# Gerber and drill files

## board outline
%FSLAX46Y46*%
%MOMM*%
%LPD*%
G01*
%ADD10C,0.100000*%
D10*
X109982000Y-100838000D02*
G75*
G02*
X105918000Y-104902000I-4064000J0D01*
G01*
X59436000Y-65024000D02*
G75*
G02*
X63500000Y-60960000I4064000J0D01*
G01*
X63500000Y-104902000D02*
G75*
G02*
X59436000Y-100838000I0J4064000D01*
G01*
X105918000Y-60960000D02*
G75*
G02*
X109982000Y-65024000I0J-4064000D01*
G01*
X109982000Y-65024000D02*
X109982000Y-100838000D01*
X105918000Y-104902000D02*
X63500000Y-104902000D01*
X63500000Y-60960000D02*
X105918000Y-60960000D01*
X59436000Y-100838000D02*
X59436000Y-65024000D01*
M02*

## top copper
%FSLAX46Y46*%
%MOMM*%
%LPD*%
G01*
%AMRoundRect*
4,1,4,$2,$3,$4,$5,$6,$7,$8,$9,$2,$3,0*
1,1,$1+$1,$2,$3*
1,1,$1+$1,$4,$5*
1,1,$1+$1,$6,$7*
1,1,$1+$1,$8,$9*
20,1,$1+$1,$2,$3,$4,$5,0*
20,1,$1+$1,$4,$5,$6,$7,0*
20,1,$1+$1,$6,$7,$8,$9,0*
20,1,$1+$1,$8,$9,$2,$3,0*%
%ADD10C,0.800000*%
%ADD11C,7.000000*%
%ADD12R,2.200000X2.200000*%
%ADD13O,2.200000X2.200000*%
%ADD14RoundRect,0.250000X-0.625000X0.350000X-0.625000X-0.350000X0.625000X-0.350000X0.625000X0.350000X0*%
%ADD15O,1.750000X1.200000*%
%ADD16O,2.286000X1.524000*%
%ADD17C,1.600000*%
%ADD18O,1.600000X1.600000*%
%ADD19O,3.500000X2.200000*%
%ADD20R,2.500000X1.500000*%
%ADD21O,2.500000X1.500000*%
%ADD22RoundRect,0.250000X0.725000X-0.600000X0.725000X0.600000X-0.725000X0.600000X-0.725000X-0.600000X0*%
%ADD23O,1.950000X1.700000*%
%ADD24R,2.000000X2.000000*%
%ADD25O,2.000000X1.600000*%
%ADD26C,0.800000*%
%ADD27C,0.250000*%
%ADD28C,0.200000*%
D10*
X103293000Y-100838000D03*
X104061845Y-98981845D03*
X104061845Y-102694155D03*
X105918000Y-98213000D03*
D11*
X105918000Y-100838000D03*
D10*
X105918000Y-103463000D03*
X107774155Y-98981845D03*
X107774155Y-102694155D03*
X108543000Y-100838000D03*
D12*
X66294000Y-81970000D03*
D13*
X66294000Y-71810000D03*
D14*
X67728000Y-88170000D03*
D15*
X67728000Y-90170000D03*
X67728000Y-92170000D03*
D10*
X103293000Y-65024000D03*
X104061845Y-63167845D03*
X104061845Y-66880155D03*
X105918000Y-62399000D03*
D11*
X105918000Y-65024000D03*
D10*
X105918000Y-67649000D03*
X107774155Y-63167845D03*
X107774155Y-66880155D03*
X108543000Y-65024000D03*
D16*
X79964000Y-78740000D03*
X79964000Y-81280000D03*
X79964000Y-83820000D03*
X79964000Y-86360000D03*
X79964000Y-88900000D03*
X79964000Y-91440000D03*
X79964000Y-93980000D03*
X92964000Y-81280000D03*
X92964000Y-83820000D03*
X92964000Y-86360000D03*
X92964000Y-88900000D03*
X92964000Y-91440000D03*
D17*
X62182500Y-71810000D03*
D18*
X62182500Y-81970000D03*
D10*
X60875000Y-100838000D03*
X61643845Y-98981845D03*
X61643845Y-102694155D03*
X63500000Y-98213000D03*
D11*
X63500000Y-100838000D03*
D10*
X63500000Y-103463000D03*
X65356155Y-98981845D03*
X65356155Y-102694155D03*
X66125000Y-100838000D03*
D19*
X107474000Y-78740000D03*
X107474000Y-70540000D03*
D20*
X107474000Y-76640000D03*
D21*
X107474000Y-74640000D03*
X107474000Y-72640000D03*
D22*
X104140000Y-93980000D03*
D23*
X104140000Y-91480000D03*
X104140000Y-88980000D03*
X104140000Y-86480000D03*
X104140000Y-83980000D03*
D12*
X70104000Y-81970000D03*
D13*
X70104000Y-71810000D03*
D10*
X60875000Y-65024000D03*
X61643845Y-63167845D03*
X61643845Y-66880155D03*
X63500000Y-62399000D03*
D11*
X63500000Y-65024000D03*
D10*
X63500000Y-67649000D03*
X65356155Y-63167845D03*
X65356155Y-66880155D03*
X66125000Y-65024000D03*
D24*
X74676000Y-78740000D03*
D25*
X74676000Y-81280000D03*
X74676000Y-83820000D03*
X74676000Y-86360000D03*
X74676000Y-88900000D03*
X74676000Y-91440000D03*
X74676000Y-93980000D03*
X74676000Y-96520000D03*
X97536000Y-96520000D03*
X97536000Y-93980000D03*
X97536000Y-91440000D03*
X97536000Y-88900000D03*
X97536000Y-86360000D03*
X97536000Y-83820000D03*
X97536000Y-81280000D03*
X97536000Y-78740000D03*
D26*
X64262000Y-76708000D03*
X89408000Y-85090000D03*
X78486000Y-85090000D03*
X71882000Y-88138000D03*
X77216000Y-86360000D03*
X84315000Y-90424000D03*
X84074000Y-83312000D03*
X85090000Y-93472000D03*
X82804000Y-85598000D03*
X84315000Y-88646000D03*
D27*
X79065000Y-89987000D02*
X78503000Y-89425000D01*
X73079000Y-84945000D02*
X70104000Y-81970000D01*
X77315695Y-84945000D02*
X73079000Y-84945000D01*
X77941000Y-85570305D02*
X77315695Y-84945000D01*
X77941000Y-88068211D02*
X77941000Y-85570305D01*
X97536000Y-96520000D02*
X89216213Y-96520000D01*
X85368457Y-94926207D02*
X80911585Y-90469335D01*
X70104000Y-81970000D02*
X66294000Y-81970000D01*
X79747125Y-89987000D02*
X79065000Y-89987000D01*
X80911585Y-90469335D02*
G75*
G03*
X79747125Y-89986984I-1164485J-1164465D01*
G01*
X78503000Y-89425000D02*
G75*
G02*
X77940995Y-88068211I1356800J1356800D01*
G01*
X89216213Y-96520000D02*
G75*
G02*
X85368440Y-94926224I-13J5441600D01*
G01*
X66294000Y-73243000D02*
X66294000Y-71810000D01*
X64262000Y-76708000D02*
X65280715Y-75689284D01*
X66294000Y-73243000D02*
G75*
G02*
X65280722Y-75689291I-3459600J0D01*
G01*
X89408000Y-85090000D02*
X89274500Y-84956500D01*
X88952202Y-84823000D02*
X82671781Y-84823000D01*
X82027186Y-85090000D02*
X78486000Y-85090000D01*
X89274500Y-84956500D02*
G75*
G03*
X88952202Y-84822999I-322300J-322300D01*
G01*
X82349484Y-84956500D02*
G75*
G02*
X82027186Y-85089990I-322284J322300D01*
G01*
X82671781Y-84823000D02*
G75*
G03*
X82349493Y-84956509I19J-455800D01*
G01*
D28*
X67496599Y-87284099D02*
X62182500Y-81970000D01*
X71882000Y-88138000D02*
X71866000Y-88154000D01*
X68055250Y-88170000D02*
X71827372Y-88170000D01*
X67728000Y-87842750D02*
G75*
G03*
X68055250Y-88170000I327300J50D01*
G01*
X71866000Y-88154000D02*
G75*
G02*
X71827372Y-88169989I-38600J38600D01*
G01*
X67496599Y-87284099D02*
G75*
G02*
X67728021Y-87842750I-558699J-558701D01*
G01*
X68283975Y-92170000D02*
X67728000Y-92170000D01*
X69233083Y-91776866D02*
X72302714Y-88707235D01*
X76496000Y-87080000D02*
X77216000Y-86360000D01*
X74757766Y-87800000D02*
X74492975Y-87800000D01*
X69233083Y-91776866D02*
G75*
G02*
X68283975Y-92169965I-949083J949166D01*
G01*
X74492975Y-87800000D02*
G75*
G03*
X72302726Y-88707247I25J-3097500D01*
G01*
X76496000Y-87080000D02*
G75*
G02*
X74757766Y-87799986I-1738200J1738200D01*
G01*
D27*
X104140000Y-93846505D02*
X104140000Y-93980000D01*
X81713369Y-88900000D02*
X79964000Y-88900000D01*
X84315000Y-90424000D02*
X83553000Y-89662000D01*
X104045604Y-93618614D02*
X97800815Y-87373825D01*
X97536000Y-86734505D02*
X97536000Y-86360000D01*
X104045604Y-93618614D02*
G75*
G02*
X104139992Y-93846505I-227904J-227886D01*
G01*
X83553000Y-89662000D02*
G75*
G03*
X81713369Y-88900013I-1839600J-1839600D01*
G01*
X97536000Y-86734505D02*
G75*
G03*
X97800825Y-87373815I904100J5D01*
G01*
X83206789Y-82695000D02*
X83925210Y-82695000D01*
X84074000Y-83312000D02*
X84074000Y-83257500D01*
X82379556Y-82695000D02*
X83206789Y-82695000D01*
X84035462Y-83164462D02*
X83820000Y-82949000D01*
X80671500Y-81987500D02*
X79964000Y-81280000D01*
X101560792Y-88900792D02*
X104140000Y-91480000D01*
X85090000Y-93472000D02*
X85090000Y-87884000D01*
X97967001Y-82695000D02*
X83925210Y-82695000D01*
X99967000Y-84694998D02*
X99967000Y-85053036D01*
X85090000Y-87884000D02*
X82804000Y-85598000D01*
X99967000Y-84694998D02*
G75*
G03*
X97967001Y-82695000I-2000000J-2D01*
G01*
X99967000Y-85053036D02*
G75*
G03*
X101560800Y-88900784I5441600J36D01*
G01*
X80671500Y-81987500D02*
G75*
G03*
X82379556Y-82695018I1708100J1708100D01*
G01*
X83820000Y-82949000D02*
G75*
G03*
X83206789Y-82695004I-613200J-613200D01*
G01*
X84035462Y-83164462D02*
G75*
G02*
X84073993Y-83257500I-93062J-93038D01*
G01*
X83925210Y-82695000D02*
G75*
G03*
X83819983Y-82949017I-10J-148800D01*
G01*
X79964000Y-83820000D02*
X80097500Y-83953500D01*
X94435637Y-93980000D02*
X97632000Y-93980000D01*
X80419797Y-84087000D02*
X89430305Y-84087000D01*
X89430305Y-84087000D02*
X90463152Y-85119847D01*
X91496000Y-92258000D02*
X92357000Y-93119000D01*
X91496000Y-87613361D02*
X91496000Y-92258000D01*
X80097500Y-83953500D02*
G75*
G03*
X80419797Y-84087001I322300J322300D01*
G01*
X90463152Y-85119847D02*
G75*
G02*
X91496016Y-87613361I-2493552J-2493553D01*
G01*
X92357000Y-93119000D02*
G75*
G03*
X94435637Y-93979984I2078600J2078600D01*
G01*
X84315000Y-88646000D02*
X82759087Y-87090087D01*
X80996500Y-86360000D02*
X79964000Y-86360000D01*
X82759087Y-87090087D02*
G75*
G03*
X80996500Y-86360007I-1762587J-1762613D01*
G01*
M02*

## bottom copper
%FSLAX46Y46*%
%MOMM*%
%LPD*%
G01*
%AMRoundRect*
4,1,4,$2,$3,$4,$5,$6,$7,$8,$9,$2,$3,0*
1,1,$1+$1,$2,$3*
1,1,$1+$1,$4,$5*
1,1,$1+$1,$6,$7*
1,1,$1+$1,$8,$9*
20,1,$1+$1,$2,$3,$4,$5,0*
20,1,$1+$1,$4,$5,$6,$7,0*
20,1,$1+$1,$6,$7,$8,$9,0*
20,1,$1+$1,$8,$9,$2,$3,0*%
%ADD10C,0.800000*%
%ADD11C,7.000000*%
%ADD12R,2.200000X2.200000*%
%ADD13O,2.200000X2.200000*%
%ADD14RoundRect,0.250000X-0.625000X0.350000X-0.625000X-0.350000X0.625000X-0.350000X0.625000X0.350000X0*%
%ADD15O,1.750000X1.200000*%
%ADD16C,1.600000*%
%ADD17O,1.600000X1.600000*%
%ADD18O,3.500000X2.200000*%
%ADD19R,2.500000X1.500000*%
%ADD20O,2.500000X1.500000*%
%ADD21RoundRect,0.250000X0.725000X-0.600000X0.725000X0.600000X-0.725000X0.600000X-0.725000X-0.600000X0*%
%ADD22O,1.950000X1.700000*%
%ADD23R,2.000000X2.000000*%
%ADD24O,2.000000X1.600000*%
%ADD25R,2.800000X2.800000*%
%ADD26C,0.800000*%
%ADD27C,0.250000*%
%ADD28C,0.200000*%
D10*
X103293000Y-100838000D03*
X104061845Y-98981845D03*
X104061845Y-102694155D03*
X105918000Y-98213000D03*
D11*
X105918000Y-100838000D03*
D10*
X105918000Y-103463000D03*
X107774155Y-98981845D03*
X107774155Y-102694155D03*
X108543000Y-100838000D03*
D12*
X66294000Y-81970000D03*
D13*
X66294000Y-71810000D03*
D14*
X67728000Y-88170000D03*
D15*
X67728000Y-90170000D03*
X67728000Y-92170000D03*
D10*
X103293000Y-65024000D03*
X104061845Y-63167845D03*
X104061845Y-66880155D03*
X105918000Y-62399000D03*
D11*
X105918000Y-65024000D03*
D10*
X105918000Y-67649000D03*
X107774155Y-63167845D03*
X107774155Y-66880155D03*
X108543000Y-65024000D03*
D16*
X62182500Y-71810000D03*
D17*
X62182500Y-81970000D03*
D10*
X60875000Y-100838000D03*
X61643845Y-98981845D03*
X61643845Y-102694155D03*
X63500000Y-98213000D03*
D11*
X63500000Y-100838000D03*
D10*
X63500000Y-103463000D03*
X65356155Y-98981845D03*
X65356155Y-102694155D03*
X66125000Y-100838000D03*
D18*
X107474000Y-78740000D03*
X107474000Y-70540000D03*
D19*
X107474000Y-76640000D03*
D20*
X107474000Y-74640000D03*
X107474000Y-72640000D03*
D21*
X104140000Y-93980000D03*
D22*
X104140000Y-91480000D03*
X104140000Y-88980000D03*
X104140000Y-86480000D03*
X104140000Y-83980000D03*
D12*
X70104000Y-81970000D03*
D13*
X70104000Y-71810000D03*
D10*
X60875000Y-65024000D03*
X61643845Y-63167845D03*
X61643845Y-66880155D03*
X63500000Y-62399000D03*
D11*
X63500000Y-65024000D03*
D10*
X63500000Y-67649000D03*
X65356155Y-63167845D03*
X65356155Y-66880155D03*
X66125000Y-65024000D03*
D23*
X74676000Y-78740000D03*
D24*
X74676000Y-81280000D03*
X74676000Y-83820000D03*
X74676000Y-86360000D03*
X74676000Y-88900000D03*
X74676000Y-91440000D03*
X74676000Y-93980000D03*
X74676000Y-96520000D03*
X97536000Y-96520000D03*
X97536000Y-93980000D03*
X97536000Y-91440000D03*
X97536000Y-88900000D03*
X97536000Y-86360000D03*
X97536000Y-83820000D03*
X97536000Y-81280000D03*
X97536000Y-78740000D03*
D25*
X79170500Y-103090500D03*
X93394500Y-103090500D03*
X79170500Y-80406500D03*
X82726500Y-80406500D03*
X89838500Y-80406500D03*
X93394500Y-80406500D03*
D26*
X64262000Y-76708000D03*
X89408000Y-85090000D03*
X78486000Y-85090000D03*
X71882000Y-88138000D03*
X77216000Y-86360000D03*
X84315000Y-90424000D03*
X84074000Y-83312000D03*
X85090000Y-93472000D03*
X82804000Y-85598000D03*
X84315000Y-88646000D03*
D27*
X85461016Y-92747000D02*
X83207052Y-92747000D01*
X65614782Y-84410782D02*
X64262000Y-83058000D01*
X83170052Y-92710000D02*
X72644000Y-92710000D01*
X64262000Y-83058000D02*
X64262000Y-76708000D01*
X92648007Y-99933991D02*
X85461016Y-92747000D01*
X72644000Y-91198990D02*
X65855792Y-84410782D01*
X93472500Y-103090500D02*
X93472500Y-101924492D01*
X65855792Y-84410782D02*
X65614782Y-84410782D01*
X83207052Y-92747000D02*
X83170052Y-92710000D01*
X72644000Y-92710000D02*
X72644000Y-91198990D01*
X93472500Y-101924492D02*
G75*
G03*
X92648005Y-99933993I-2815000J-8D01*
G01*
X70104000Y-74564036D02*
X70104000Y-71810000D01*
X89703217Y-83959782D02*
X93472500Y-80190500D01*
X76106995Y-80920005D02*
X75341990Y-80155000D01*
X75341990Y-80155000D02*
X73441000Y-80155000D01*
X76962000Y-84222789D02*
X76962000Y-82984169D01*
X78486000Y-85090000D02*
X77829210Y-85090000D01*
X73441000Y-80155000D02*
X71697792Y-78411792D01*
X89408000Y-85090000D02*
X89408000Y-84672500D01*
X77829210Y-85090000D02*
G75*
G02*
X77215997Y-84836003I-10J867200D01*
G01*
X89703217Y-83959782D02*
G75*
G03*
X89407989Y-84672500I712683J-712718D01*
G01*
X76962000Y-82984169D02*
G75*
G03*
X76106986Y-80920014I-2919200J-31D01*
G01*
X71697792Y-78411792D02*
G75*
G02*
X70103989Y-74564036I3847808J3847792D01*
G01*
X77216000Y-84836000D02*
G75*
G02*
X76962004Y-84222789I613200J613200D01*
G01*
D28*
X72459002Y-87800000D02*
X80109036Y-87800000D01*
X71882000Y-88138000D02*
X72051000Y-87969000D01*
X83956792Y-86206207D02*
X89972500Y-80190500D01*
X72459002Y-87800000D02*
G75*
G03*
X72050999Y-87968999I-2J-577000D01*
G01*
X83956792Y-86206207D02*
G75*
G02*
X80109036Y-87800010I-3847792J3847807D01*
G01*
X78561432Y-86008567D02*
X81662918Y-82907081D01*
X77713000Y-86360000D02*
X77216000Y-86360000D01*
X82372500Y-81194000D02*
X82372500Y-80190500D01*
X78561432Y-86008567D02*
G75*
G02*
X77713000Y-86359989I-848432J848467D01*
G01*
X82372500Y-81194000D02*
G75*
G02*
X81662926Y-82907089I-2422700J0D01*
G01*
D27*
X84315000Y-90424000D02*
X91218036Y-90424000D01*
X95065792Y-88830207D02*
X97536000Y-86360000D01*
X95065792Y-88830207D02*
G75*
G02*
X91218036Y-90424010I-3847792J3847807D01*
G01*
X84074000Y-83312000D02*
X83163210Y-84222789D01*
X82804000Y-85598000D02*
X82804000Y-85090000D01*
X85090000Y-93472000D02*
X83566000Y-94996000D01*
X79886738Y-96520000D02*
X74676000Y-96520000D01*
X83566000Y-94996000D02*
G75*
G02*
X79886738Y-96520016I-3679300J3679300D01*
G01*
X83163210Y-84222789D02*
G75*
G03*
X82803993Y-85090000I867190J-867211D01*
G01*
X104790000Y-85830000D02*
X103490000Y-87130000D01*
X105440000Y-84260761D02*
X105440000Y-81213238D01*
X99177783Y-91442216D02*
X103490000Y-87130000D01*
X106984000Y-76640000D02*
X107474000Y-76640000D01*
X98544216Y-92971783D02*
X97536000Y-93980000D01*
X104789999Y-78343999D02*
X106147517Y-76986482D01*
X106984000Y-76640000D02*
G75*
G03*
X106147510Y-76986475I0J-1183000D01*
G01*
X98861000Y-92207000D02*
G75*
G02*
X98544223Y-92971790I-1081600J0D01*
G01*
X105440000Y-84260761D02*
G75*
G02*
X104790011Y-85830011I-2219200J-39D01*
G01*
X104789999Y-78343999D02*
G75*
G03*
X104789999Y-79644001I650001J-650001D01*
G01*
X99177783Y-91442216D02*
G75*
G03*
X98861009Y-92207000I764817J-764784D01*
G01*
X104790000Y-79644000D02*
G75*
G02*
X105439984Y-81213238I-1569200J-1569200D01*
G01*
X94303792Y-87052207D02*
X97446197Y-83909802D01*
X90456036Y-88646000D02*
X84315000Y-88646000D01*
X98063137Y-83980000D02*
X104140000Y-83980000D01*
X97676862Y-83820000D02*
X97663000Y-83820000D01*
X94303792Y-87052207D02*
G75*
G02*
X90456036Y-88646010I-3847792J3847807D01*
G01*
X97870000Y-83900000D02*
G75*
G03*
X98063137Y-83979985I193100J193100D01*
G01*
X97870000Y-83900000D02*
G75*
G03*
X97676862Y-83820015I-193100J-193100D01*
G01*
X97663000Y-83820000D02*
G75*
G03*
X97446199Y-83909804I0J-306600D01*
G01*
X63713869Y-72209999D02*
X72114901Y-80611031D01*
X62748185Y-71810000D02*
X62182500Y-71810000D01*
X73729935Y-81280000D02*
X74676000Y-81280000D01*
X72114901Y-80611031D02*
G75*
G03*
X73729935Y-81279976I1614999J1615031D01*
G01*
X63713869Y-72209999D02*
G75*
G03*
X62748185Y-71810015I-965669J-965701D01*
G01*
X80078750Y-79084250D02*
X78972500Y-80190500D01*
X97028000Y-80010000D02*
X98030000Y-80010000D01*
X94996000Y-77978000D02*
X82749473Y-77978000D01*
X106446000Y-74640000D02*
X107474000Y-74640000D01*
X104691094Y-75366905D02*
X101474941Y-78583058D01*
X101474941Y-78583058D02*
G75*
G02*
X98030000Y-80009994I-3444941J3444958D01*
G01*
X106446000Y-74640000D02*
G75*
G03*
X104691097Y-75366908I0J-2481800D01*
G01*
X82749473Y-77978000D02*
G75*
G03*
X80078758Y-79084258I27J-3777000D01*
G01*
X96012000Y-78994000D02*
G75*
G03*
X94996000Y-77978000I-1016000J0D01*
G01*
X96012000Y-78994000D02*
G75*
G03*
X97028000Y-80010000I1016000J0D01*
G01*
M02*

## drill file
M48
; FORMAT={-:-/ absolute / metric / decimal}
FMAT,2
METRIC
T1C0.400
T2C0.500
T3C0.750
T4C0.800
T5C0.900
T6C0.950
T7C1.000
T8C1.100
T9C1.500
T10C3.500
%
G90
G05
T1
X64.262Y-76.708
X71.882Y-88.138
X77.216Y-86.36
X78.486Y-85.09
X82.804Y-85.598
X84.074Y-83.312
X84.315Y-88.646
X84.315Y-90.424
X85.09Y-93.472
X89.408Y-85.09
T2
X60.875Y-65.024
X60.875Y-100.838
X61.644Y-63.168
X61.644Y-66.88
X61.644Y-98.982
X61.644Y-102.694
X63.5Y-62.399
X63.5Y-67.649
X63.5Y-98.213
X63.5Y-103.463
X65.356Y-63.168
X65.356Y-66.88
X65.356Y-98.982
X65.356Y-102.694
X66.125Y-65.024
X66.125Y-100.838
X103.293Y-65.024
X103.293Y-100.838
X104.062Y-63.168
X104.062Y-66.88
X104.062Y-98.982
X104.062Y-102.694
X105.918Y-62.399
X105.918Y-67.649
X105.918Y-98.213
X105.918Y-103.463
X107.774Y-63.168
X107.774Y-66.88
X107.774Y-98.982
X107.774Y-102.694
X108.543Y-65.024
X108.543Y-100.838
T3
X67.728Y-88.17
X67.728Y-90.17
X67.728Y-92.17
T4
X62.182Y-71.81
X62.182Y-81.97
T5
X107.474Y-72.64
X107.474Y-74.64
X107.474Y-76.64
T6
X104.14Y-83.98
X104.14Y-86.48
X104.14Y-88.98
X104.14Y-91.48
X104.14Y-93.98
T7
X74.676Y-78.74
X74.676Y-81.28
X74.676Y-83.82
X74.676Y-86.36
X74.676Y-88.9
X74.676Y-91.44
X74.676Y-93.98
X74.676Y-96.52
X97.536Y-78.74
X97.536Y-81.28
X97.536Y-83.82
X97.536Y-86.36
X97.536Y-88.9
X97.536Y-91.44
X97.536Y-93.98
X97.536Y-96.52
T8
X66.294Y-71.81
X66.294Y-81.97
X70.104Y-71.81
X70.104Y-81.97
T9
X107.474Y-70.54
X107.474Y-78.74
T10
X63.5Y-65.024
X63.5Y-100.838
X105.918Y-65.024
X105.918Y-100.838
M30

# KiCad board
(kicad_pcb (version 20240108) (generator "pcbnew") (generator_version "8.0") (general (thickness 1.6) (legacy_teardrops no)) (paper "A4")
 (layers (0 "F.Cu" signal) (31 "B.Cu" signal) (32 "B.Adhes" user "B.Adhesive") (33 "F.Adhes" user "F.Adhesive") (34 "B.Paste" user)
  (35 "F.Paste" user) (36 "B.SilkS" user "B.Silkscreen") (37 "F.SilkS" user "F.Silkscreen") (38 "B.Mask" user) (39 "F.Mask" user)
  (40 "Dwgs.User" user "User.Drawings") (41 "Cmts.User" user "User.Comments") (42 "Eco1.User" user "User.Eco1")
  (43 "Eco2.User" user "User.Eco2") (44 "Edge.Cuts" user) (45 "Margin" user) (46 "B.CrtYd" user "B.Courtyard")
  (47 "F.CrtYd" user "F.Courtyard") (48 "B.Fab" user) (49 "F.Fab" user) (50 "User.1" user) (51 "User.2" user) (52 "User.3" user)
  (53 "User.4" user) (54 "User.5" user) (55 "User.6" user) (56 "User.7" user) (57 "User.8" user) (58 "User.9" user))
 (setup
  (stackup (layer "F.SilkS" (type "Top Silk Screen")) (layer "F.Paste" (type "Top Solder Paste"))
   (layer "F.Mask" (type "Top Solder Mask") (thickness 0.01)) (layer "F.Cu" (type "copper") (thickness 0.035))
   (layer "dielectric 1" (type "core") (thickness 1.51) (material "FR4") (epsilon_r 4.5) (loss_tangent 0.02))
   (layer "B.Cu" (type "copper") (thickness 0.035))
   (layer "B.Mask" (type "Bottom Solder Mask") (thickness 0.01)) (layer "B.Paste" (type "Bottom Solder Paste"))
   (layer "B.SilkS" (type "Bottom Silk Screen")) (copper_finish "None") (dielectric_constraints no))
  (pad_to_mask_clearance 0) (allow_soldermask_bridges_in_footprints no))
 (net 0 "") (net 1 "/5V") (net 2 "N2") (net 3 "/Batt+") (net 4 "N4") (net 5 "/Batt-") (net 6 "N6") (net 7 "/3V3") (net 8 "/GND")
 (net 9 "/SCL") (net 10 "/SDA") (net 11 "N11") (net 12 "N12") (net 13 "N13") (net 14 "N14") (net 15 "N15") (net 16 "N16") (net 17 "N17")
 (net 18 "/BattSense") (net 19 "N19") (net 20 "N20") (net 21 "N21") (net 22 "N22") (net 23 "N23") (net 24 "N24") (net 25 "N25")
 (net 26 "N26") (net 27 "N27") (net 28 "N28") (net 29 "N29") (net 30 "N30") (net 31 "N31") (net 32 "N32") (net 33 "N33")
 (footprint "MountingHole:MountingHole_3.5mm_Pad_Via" (layer "F.Cu") (at 105.918 100.838)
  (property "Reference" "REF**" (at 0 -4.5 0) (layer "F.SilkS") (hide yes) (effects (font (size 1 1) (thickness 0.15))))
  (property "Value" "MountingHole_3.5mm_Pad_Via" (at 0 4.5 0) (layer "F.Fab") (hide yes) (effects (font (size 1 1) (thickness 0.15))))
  (pad "1" thru_hole circle (at -2.625 0) (size 0.8 0.8) (drill 0.5) (layers "*.Cu" "*.Mask") (remove_unused_layers no) (zone_connect 2))
  (pad "1" thru_hole circle (at -1.856155 -1.856155) (size 0.8 0.8) (drill 0.5) (layers "*.Cu" "*.Mask") (remove_unused_layers no)
   (zone_connect 2))
  (pad "1" thru_hole circle (at -1.856155 1.856155) (size 0.8 0.8) (drill 0.5) (layers "*.Cu" "*.Mask") (remove_unused_layers no)
   (zone_connect 2))
  (pad "1" thru_hole circle (at 0 -2.625) (size 0.8 0.8) (drill 0.5) (layers "*.Cu" "*.Mask") (remove_unused_layers no) (zone_connect 2))
  (pad "1" thru_hole circle (at 0 0) (size 7 7) (drill 3.5) (layers "*.Cu" "*.Mask") (remove_unused_layers no))
  (pad "1" thru_hole circle (at 0 2.625) (size 0.8 0.8) (drill 0.5) (layers "*.Cu" "*.Mask") (remove_unused_layers no) (zone_connect 2))
  (pad "1" thru_hole circle (at 1.856155 -1.856155) (size 0.8 0.8) (drill 0.5) (layers "*.Cu" "*.Mask") (remove_unused_layers no)
   (zone_connect 2))
  (pad "1" thru_hole circle (at 1.856155 1.856155) (size 0.8 0.8) (drill 0.5) (layers "*.Cu" "*.Mask") (remove_unused_layers no)
   (zone_connect 2))
  (pad "1" thru_hole circle (at 2.625 0) (size 0.8 0.8) (drill 0.5) (layers "*.Cu" "*.Mask") (remove_unused_layers no) (zone_connect 2)))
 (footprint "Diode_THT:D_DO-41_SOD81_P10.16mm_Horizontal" (layer "F.Cu") (at 66.294 81.97 90)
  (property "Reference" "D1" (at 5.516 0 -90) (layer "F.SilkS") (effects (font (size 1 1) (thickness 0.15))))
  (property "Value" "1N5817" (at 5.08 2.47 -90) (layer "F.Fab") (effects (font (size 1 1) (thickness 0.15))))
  (pad "1" thru_hole rect (at 0 0 90) (size 2.2 2.2) (drill 1.1) (layers "*.Cu" "*.Mask") (remove_unused_layers no) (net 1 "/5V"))
  (pad "2" thru_hole oval (at 10.16 0 90) (size 2.2 2.2) (drill 1.1) (layers "*.Cu" "*.Mask") (remove_unused_layers no) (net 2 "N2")))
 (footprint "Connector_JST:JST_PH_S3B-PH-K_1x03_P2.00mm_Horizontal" (layer "F.Cu") (at 67.728 88.17 -90)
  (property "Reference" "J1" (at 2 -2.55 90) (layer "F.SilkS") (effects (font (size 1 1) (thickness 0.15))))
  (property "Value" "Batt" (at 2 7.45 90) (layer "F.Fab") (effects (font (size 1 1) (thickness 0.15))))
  (pad "1" thru_hole roundrect (at 0 0 270) (size 1.2 1.75) (drill 0.75) (layers "*.Cu" "*.Mask") (remove_unused_layers no)
   (roundrect_rratio 0.2083333333) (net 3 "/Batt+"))
  (pad "2" thru_hole oval (at 2 0 270) (size 1.2 1.75) (drill 0.75) (layers "*.Cu" "*.Mask") (remove_unused_layers no) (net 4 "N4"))
  (pad "3" thru_hole oval (at 4 0 270) (size 1.2 1.75) (drill 0.75) (layers "*.Cu" "*.Mask") (remove_unused_layers no) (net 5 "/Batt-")))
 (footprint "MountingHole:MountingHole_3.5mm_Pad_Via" (layer "F.Cu") (at 105.918 65.024)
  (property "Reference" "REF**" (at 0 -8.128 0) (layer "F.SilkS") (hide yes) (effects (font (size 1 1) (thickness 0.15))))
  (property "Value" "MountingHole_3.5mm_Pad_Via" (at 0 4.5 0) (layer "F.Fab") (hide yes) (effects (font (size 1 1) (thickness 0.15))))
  (pad "1" thru_hole circle (at -2.625 0) (size 0.8 0.8) (drill 0.5) (layers "*.Cu" "*.Mask") (remove_unused_layers no) (zone_connect 2))
  (pad "1" thru_hole circle (at -1.856155 -1.856155) (size 0.8 0.8) (drill 0.5) (layers "*.Cu" "*.Mask") (remove_unused_layers no)
   (zone_connect 2))
  (pad "1" thru_hole circle (at -1.856155 1.856155) (size 0.8 0.8) (drill 0.5) (layers "*.Cu" "*.Mask") (remove_unused_layers no)
   (zone_connect 2))
  (pad "1" thru_hole circle (at 0 -2.625) (size 0.8 0.8) (drill 0.5) (layers "*.Cu" "*.Mask") (remove_unused_layers no) (zone_connect 2))
  (pad "1" thru_hole circle (at 0 0) (size 7 7) (drill 3.5) (layers "*.Cu" "*.Mask") (remove_unused_layers no))
  (pad "1" thru_hole circle (at 0 2.625) (size 0.8 0.8) (drill 0.5) (layers "*.Cu" "*.Mask") (remove_unused_layers no) (zone_connect 2))
  (pad "1" thru_hole circle (at 1.856155 -1.856155) (size 0.8 0.8) (drill 0.5) (layers "*.Cu" "*.Mask") (remove_unused_layers no)
   (zone_connect 2))
  (pad "1" thru_hole circle (at 1.856155 1.856155) (size 0.8 0.8) (drill 0.5) (layers "*.Cu" "*.Mask") (remove_unused_layers no)
   (zone_connect 2))
  (pad "1" thru_hole circle (at 2.625 0) (size 0.8 0.8) (drill 0.5) (layers "*.Cu" "*.Mask") (remove_unused_layers no) (zone_connect 2)))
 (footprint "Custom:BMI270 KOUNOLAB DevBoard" (layer "F.Cu") (at 86.464 86.36)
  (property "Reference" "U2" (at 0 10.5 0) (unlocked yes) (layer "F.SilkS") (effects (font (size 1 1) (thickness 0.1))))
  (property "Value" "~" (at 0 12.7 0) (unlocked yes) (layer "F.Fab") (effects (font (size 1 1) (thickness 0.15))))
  (pad "1" smd oval (at -6.5 -7.62) (size 2.286 1.524) (layers "F.Cu" "F.Paste" "F.Mask") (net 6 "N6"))
  (pad "2" smd oval (at -6.5 -5.08) (size 2.286 1.524) (layers "F.Cu" "F.Paste" "F.Mask") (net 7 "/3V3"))
  (pad "3" smd oval (at -6.5 -2.54) (size 2.286 1.524) (layers "F.Cu" "F.Paste" "F.Mask") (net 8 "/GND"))
  (pad "4" smd oval (at -6.5 0) (size 2.286 1.524) (layers "F.Cu" "F.Paste" "F.Mask") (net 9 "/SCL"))
  (pad "5" smd oval (at -6.5 2.54) (size 2.286 1.524) (layers "F.Cu" "F.Paste" "F.Mask") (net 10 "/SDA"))
  (pad "6" smd oval (at -6.5 5.08) (size 2.286 1.524) (layers "F.Cu" "F.Paste" "F.Mask") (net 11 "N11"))
  (pad "7" smd oval (at -6.5 7.62) (size 2.286 1.524) (layers "F.Cu" "F.Paste" "F.Mask") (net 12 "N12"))
  (pad "8" smd oval (at 6.5 -5.08) (size 2.286 1.524) (layers "F.Cu" "F.Paste" "F.Mask") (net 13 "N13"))
  (pad "9" smd oval (at 6.5 -2.54) (size 2.286 1.524) (layers "F.Cu" "F.Paste" "F.Mask") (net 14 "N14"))
  (pad "10" smd oval (at 6.5 0) (size 2.286 1.524) (layers "F.Cu" "F.Paste" "F.Mask") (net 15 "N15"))
  (pad "11" smd oval (at 6.5 2.54) (size 2.286 1.524) (layers "F.Cu" "F.Paste" "F.Mask") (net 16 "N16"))
  (pad "12" smd oval (at 6.5 5.08) (size 2.286 1.524) (layers "F.Cu" "F.Paste" "F.Mask") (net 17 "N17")))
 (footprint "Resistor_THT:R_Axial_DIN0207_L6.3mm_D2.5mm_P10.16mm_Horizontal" (layer "F.Cu") (at 62.1825 71.81 -90)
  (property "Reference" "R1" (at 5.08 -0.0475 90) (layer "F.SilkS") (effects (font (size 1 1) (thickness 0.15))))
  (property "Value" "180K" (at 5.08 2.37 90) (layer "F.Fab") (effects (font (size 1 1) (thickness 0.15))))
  (pad "1" thru_hole circle (at 0 0 270) (size 1.6 1.6) (drill 0.8) (layers "*.Cu" "*.Mask") (remove_unused_layers no) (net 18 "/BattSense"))
  (pad "2" thru_hole oval (at 10.16 0 270) (size 1.6 1.6) (drill 0.8) (layers "*.Cu" "*.Mask") (remove_unused_layers no) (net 3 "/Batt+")))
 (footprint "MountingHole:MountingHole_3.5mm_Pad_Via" (layer "F.Cu") (at 63.5 100.838)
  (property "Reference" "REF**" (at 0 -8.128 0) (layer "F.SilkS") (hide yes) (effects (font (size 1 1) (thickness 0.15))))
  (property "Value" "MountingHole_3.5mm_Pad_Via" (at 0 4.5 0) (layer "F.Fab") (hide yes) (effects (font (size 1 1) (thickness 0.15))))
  (pad "1" thru_hole circle (at -2.625 0) (size 0.8 0.8) (drill 0.5) (layers "*.Cu" "*.Mask") (remove_unused_layers no) (zone_connect 2))
  (pad "1" thru_hole circle (at -1.856155 -1.856155) (size 0.8 0.8) (drill 0.5) (layers "*.Cu" "*.Mask") (remove_unused_layers no)
   (zone_connect 2))
  (pad "1" thru_hole circle (at -1.856155 1.856155) (size 0.8 0.8) (drill 0.5) (layers "*.Cu" "*.Mask") (remove_unused_layers no)
   (zone_connect 2))
  (pad "1" thru_hole circle (at 0 -2.625) (size 0.8 0.8) (drill 0.5) (layers "*.Cu" "*.Mask") (remove_unused_layers no) (zone_connect 2))
  (pad "1" thru_hole circle (at 0 0) (size 7 7) (drill 3.5) (layers "*.Cu" "*.Mask") (remove_unused_layers no))
  (pad "1" thru_hole circle (at 0 2.625) (size 0.8 0.8) (drill 0.5) (layers "*.Cu" "*.Mask") (remove_unused_layers no) (zone_connect 2))
  (pad "1" thru_hole circle (at 1.856155 -1.856155) (size 0.8 0.8) (drill 0.5) (layers "*.Cu" "*.Mask") (remove_unused_layers no)
   (zone_connect 2))
  (pad "1" thru_hole circle (at 1.856155 1.856155) (size 0.8 0.8) (drill 0.5) (layers "*.Cu" "*.Mask") (remove_unused_layers no)
   (zone_connect 2))
  (pad "1" thru_hole circle (at 2.625 0) (size 0.8 0.8) (drill 0.5) (layers "*.Cu" "*.Mask") (remove_unused_layers no) (zone_connect 2)))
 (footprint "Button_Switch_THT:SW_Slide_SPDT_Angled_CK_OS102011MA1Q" (layer "F.Cu") (at 107.474 76.64 90)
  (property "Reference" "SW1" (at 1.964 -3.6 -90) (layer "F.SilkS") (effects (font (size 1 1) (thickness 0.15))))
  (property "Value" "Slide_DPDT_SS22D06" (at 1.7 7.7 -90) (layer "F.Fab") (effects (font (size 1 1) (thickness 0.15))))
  (pad "" thru_hole oval (at -2.1 0 90) (size 2.2 3.5) (drill 1.5) (layers "*.Cu" "*.Mask") (remove_unused_layers no))
  (pad "" thru_hole oval (at 6.1 0 90) (size 2.2 3.5) (drill 1.5) (layers "*.Cu" "*.Mask") (remove_unused_layers no))
  (pad "1" thru_hole rect (at 0 0 90) (size 1.5 2.5) (drill 0.9) (layers "*.Cu" "*.Mask") (remove_unused_layers no) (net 8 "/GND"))
  (pad "2" thru_hole oval (at 2 0 90) (size 1.5 2.5) (drill 0.9) (layers "*.Cu" "*.Mask") (remove_unused_layers no) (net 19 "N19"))
  (pad "3" thru_hole oval (at 4 0 90) (size 1.5 2.5) (drill 0.9) (layers "*.Cu" "*.Mask") (remove_unused_layers no) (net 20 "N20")))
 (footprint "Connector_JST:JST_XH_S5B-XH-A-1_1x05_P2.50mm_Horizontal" (layer "F.Cu") (at 104.14 93.98 90)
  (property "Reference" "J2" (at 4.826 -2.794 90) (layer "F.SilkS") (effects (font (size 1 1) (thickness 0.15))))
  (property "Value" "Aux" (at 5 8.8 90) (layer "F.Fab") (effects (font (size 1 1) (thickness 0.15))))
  (pad "1" thru_hole roundrect (at 0 0 90) (size 1.7 1.95) (drill 0.95) (layers "*.Cu" "*.Mask") (remove_unused_layers no)
   (roundrect_rratio 0.1470588235) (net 10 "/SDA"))
  (pad "2" thru_hole oval (at 2.5 0 90) (size 1.7 1.95) (drill 0.95) (layers "*.Cu" "*.Mask") (remove_unused_layers no) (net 7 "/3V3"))
  (pad "3" thru_hole oval (at 5 0 90) (size 1.7 1.95) (drill 0.95) (layers "*.Cu" "*.Mask") (remove_unused_layers no) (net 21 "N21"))
  (pad "4" thru_hole oval (at 7.5 0 90) (size 1.7 1.95) (drill 0.95) (layers "*.Cu" "*.Mask") (remove_unused_layers no) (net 8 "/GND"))
  (pad "5" thru_hole oval (at 10 0 90) (size 1.7 1.95) (drill 0.95) (layers "*.Cu" "*.Mask") (remove_unused_layers no) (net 9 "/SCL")))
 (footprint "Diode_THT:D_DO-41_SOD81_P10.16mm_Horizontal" (layer "F.Cu") (at 70.104 81.97 90)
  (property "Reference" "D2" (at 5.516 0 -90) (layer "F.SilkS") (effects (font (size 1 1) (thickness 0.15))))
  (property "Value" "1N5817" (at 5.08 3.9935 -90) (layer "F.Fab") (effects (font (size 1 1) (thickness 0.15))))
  (pad "1" thru_hole rect (at 0 0 90) (size 2.2 2.2) (drill 1.1) (layers "*.Cu" "*.Mask") (remove_unused_layers no) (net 1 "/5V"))
  (pad "2" thru_hole oval (at 10.16 0 90) (size 2.2 2.2) (drill 1.1) (layers "*.Cu" "*.Mask") (remove_unused_layers no) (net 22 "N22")))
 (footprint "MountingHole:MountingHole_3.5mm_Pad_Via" (layer "F.Cu") (at 63.5 65.024)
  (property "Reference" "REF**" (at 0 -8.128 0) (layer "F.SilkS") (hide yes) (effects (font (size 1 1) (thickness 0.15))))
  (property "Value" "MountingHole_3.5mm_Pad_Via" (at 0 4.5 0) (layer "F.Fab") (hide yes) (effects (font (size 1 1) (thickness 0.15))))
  (pad "1" thru_hole circle (at -2.625 0) (size 0.8 0.8) (drill 0.5) (layers "*.Cu" "*.Mask") (remove_unused_layers no) (zone_connect 2))
  (pad "1" thru_hole circle (at -1.856155 -1.856155) (size 0.8 0.8) (drill 0.5) (layers "*.Cu" "*.Mask") (remove_unused_layers no)
   (zone_connect 2))
  (pad "1" thru_hole circle (at -1.856155 1.856155) (size 0.8 0.8) (drill 0.5) (layers "*.Cu" "*.Mask") (remove_unused_layers no)
   (zone_connect 2))
  (pad "1" thru_hole circle (at 0 -2.625) (size 0.8 0.8) (drill 0.5) (layers "*.Cu" "*.Mask") (remove_unused_layers no) (zone_connect 2))
  (pad "1" thru_hole circle (at 0 0) (size 7 7) (drill 3.5) (layers "*.Cu" "*.Mask") (remove_unused_layers no))
  (pad "1" thru_hole circle (at 0 2.625) (size 0.8 0.8) (drill 0.5) (layers "*.Cu" "*.Mask") (remove_unused_layers no) (zone_connect 2))
  (pad "1" thru_hole circle (at 1.856155 -1.856155) (size 0.8 0.8) (drill 0.5) (layers "*.Cu" "*.Mask") (remove_unused_layers no)
   (zone_connect 2))
  (pad "1" thru_hole circle (at 1.856155 1.856155) (size 0.8 0.8) (drill 0.5) (layers "*.Cu" "*.Mask") (remove_unused_layers no)
   (zone_connect 2))
  (pad "1" thru_hole circle (at 2.625 0) (size 0.8 0.8) (drill 0.5) (layers "*.Cu" "*.Mask") (remove_unused_layers no) (zone_connect 2)))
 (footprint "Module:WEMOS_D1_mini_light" (layer "F.Cu") (at 74.676 78.74)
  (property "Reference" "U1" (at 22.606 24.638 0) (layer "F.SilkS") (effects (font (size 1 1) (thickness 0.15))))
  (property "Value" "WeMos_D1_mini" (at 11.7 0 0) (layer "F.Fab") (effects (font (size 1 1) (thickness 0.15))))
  (pad "1" thru_hole rect (at 0 0) (size 2 2) (drill 1) (layers "*.Cu" "*.Mask") (remove_unused_layers no) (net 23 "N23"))
  (pad "2" thru_hole oval (at 0 2.54) (size 2 1.6) (drill 1) (layers "*.Cu" "*.Mask") (remove_unused_layers no) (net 18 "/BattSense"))
  (pad "3" thru_hole oval (at 0 5.08) (size 2 1.6) (drill 1) (layers "*.Cu" "*.Mask") (remove_unused_layers no) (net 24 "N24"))
  (pad "4" thru_hole oval (at 0 7.62) (size 2 1.6) (drill 1) (layers "*.Cu" "*.Mask") (remove_unused_layers no) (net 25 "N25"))
  (pad "5" thru_hole oval (at 0 10.16) (size 2 1.6) (drill 1) (layers "*.Cu" "*.Mask") (remove_unused_layers no) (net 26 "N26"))
  (pad "6" thru_hole oval (at 0 12.7) (size 2 1.6) (drill 1) (layers "*.Cu" "*.Mask") (remove_unused_layers no) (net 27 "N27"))
  (pad "7" thru_hole oval (at 0 15.24) (size 2 1.6) (drill 1) (layers "*.Cu" "*.Mask") (remove_unused_layers no) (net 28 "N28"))
  (pad "8" thru_hole oval (at 0 17.78) (size 2 1.6) (drill 1) (layers "*.Cu" "*.Mask") (remove_unused_layers no) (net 7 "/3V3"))
  (pad "9" thru_hole oval (at 22.86 17.78) (size 2 1.6) (drill 1) (layers "*.Cu" "*.Mask") (remove_unused_layers no) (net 1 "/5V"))
  (pad "10" thru_hole oval (at 22.86 15.24) (size 2 1.6) (drill 1) (layers "*.Cu" "*.Mask") (remove_unused_layers no) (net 8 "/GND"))
  (pad "11" thru_hole oval (at 22.86 12.7) (size 2 1.6) (drill 1) (layers "*.Cu" "*.Mask") (remove_unused_layers no) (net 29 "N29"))
  (pad "12" thru_hole oval (at 22.86 10.16) (size 2 1.6) (drill 1) (layers "*.Cu" "*.Mask") (remove_unused_layers no) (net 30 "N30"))
  (pad "13" thru_hole oval (at 22.86 7.62) (size 2 1.6) (drill 1) (layers "*.Cu" "*.Mask") (remove_unused_layers no) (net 10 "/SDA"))
  (pad "14" thru_hole oval (at 22.86 5.08) (size 2 1.6) (drill 1) (layers "*.Cu" "*.Mask") (remove_unused_layers no) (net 9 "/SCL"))
  (pad "15" thru_hole oval (at 22.86 2.54) (size 2 1.6) (drill 1) (layers "*.Cu" "*.Mask") (remove_unused_layers no) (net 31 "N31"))
  (pad "16" thru_hole oval (at 22.86 0) (size 2 1.6) (drill 1) (layers "*.Cu" "*.Mask") (remove_unused_layers no) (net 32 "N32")))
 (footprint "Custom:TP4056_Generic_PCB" (layer "B.Cu") (at 95.1725 104.7905 90)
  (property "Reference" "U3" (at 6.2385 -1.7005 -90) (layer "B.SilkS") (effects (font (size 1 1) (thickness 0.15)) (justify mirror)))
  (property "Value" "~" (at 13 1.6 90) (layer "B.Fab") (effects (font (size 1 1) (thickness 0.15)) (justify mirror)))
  (pad "1" smd rect (at 1.7 -16.002 90) (size 2.8 2.8) (layers "B.Cu" "B.Paste" "B.Mask") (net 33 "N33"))
  (pad "2" smd rect (at 1.7 -1.778 90) (size 2.8 2.8) (layers "B.Cu" "B.Paste" "B.Mask") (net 2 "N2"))
  (pad "3" smd rect (at 24.384 -16.002 90) (size 2.8 2.8) (layers "B.Cu" "B.Paste" "B.Mask") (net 19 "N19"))
  (pad "4" smd rect (at 24.384 -12.446 90) (size 2.8 2.8) (layers "B.Cu" "B.Paste" "B.Mask") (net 5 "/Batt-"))
  (pad "5" smd rect (at 24.384 -5.334 90) (size 2.8 2.8) (layers "B.Cu" "B.Paste" "B.Mask") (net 3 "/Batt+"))
  (pad "6" smd rect (at 24.384 -1.778 90) (size 2.8 2.8) (layers "B.Cu" "B.Paste" "B.Mask") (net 22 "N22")))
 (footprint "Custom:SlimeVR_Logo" (layer "B.Cu") (at 85.852 68.072 180)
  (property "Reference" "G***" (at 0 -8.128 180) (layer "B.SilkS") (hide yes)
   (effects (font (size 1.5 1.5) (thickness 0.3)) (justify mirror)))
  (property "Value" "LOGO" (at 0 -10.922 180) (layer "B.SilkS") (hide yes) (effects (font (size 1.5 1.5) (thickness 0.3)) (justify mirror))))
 (gr_arc (start 109.982 100.838) (mid 108.791682 103.711682) (end 105.918 104.902) (stroke (width 0.1) (type default)) (layer "Edge.Cuts"))
 (gr_arc (start 59.436 65.024) (mid 60.626318 62.150318) (end 63.5 60.96) (stroke (width 0.1) (type default)) (layer "Edge.Cuts"))
 (gr_arc (start 63.5 104.902) (mid 60.626318 103.711682) (end 59.436 100.838) (stroke (width 0.1) (type default)) (layer "Edge.Cuts"))
 (gr_arc (start 105.918 60.96) (mid 108.791682 62.150318) (end 109.982 65.024) (stroke (width 0.1) (type default)) (layer "Edge.Cuts"))
 (gr_line (start 109.982 65.024) (end 109.982 100.838) (stroke (width 0.1) (type default)) (layer "Edge.Cuts"))
 (gr_line (start 105.918 104.902) (end 63.5 104.902) (stroke (width 0.1) (type default)) (layer "Edge.Cuts"))
 (gr_line (start 63.5 60.96) (end 105.918 60.96) (stroke (width 0.1) (type default)) (layer "Edge.Cuts"))
 (gr_line (start 59.436 100.838) (end 59.436 65.024) (stroke (width 0.1) (type default)) (layer "Edge.Cuts"))
 (segment (start 79.065 89.987) (end 78.503 89.425) (width 0.25) (layer "F.Cu") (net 1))
 (segment (start 73.079 84.945) (end 70.104 81.97) (width 0.25) (layer "F.Cu") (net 1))
 (segment (start 77.315695 84.945) (end 73.079 84.945) (width 0.25) (layer "F.Cu") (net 1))
 (segment (start 77.941 85.570305) (end 77.315695 84.945) (width 0.25) (layer "F.Cu") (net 1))
 (segment (start 77.941 88.068211) (end 77.941 85.570305) (width 0.25) (layer "F.Cu") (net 1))
 (segment (start 97.536 96.52) (end 89.216213 96.52) (width 0.25) (layer "F.Cu") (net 1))
 (segment (start 85.368457 94.926207) (end 80.911585 90.469335) (width 0.25) (layer "F.Cu") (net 1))
 (segment (start 70.104 81.97) (end 66.294 81.97) (width 0.25) (layer "F.Cu") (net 1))
 (segment (start 79.747125 89.987) (end 79.065 89.987) (width 0.25) (layer "F.Cu") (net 1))
 (arc (start 80.911585 90.469335) (mid 80.377326 90.112354) (end 79.747125 89.987) (width 0.25) (layer "F.Cu") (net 1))
 (arc (start 78.503 89.425) (mid 78.087059 88.8025) (end 77.941 88.068211) (width 0.25) (layer "F.Cu") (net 1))
 (arc (start 89.216213 96.52) (mid 87.133822 96.105786) (end 85.368457 94.926207) (width 0.25) (layer "F.Cu") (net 1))
 (segment (start 66.294 73.243) (end 66.294 71.81) (width 0.25) (layer "F.Cu") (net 2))
 (segment (start 64.262 76.708) (end 65.280715 75.689284) (width 0.25) (layer "F.Cu") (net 2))
 (via (at 64.262 76.708) (size 0.8) (drill 0.4) (layers "F.Cu" "B.Cu") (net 2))
 (arc (start 66.294 73.243) (mid 66.030655 74.566919) (end 65.280715 75.689284) (width 0.25) (layer "F.Cu") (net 2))
 (segment (start 85.461016 92.747) (end 83.207052 92.747) (width 0.25) (layer "B.Cu") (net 2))
 (segment (start 65.614782 84.410782) (end 64.262 83.058) (width 0.25) (layer "B.Cu") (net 2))
 (segment (start 83.170052 92.71) (end 72.644 92.71) (width 0.25) (layer "B.Cu") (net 2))
 (segment (start 64.262 83.058) (end 64.262 76.708) (width 0.25) (layer "B.Cu") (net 2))
 (segment (start 92.648007 99.933991) (end 85.461016 92.747) (width 0.25) (layer "B.Cu") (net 2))
 (segment (start 72.644 91.19899) (end 65.855792 84.410782) (width 0.25) (layer "B.Cu") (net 2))
 (segment (start 93.4725 103.0905) (end 93.4725 101.924492) (width 0.25) (layer "B.Cu") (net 2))
 (segment (start 65.855792 84.410782) (end 65.614782 84.410782) (width 0.25) (layer "B.Cu") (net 2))
 (segment (start 83.207052 92.747) (end 83.170052 92.71) (width 0.25) (layer "B.Cu") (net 2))
 (segment (start 72.644 92.71) (end 72.644 91.19899) (width 0.25) (layer "B.Cu") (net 2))
 (arc (start 93.4725 101.924492) (mid 93.258221 100.84724) (end 92.648007 99.933991) (width 0.25) (layer "B.Cu") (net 2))
 (segment (start 89.408 85.09) (end 89.2745 84.9565) (width 0.25) (layer "F.Cu") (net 22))
 (segment (start 88.952202 84.823) (end 82.671781 84.823) (width 0.25) (layer "F.Cu") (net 22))
 (segment (start 82.027186 85.09) (end 78.486 85.09) (width 0.25) (layer "F.Cu") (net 22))
 (via (at 89.408 85.09) (size 0.8) (drill 0.4) (layers "F.Cu" "B.Cu") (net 22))
 (via (at 78.486 85.09) (size 0.8) (drill 0.4) (layers "F.Cu" "B.Cu") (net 22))
 (arc (start 89.2745 84.9565) (mid 89.126628 84.857695) (end 88.952202 84.823) (width 0.25) (layer "F.Cu") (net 22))
 (arc (start 82.349484 84.9565) (mid 82.201612 85.055304) (end 82.027186 85.09) (width 0.25) (layer "F.Cu") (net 22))
 (arc (start 82.671781 84.823) (mid 82.497355 84.857695) (end 82.349484 84.9565) (width 0.25) (layer "F.Cu") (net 22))
 (segment (start 70.104 74.564036) (end 70.104 71.81) (width 0.25) (layer "B.Cu") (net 22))
 (segment (start 89.703217 83.959782) (end 93.4725 80.1905) (width 0.25) (layer "B.Cu") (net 22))
 (segment (start 76.106995 80.920005) (end 75.34199 80.155) (width 0.25) (layer "B.Cu") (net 22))
 (segment (start 75.34199 80.155) (end 73.441 80.155) (width 0.25) (layer "B.Cu") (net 22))
 (segment (start 76.962 84.222789) (end 76.962 82.984169) (width 0.25) (layer "B.Cu") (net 22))
 (segment (start 78.486 85.09) (end 77.82921 85.09) (width 0.25) (layer "B.Cu") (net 22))
 (segment (start 73.441 80.155) (end 71.697792 78.411792) (width 0.25) (layer "B.Cu") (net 22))
 (segment (start 89.408 85.09) (end 89.408 84.6725) (width 0.25) (layer "B.Cu") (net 22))
 (arc (start 77.82921 85.09) (mid 77.497343 85.023987) (end 77.216 84.836) (width 0.25) (layer "B.Cu") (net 22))
 (arc (start 89.703217 83.959782) (mid 89.484724 84.28678) (end 89.408 84.6725) (width 0.25) (layer "B.Cu") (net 22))
 (arc (start 76.962 82.984169) (mid 76.739791 81.867051) (end 76.106995 80.920005) (width 0.25) (layer "B.Cu") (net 22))
 (arc (start 71.697792 78.411792) (mid 70.518213 76.646426) (end 70.104 74.564036) (width 0.25) (layer "B.Cu") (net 22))
 (arc (start 77.216 84.836) (mid 77.028012 84.554656) (end 76.962 84.222789) (width 0.25) (layer "B.Cu") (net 22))
 (segment (start 67.496599 87.284099) (end 62.1825 81.97) (width 0.2) (layer "F.Cu") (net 3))
 (segment (start 71.882 88.138) (end 71.866 88.154) (width 0.2) (layer "F.Cu") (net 3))
 (segment (start 68.05525 88.17) (end 71.827372 88.17) (width 0.2) (layer "F.Cu") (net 3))
 (via (at 71.882 88.138) (size 0.8) (drill 0.4) (layers "F.Cu" "B.Cu") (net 3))
 (arc (start 67.728 87.84275) (mid 67.823849 88.07415) (end 68.05525 88.17) (width 0.2) (layer "F.Cu") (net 3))
 (arc (start 71.866 88.154) (mid 71.848277 88.165841) (end 71.827372 88.17) (width 0.2) (layer "F.Cu") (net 3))
 (arc (start 67.496599 87.284099) (mid 67.66786 87.54041) (end 67.728 87.84275) (width 0.2) (layer "F.Cu") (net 3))
 (segment (start 72.459002 87.8) (end 80.109036 87.8) (width 0.2) (layer "B.Cu") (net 3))
 (segment (start 71.882 88.138) (end 72.051 87.969) (width 0.2) (layer "B.Cu") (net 3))
 (segment (start 83.956792 86.206207) (end 89.9725 80.1905) (width 0.2) (layer "B.Cu") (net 3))
 (arc (start 72.459002 87.8) (mid 72.238192 87.843921) (end 72.051 87.969) (width 0.2) (layer "B.Cu") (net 3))
 (arc (start 83.956792 86.206207) (mid 82.191426 87.385786) (end 80.109036 87.8) (width 0.2) (layer "B.Cu") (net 3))
 (segment (start 68.283975 92.17) (end 67.728 92.17) (width 0.2) (layer "F.Cu") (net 5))
 (segment (start 69.233083 91.776866) (end 72.302714 88.707235) (width 0.2) (layer "F.Cu") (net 5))
 (segment (start 76.496 87.08) (end 77.216 86.36) (width 0.2) (layer "F.Cu") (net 5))
 (segment (start 74.757766 87.8) (end 74.492975 87.8) (width 0.2) (layer "F.Cu") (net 5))
 (via (at 77.216 86.36) (size 0.8) (drill 0.4) (layers "F.Cu" "B.Cu") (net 5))
 (arc (start 69.233083 91.776866) (mid 68.797628 92.067827) (end 68.283975 92.17) (width 0.2) (layer "F.Cu") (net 5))
 (arc (start 74.492975 87.8) (mid 73.307614 88.035782) (end 72.302714 88.707235) (width 0.2) (layer "F.Cu") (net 5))
 (arc (start 76.496 87.08) (mid 75.698491 87.612878) (end 74.757766 87.8) (width 0.2) (layer "F.Cu") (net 5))
 (segment (start 78.561432 86.008567) (end 81.662918 82.907081) (width 0.2) (layer "B.Cu") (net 5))
 (segment (start 77.713 86.36) (end 77.216 86.36) (width 0.2) (layer "B.Cu") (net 5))
 (segment (start 82.3725 81.194) (end 82.3725 80.1905) (width 0.2) (layer "B.Cu") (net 5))
 (arc (start 78.561432 86.008567) (mid 78.172168 86.268665) (end 77.713 86.36) (width 0.2) (layer "B.Cu") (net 5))
 (arc (start 82.3725 81.194) (mid 82.188085 82.121112) (end 81.662918 82.907081) (width 0.2) (layer "B.Cu") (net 5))
 (segment (start 104.14 93.846505) (end 104.14 93.98) (width 0.25) (layer "F.Cu") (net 10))
 (segment (start 81.713369 88.9) (end 79.964 88.9) (width 0.25) (layer "F.Cu") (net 10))
 (segment (start 84.315 90.424) (end 83.553 89.662) (width 0.25) (layer "F.Cu") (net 10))
 (segment (start 104.045604 93.618614) (end 97.800815 87.373825) (width 0.25) (layer "F.Cu") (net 10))
 (segment (start 97.536 86.734505) (end 97.536 86.36) (width 0.25) (layer "F.Cu") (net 10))
 (via (at 84.315 90.424) (size 0.8) (drill 0.4) (layers "F.Cu" "B.Cu") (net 10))
 (arc (start 104.045604 93.618614) (mid 104.115467 93.723171) (end 104.14 93.846505) (width 0.25) (layer "F.Cu") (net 10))
 (arc (start 83.553 89.662) (mid 82.70897 89.098037) (end 81.713369 88.9) (width 0.25) (layer "F.Cu") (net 10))
 (arc (start 97.536 86.734505) (mid 97.604823 87.080502) (end 97.800815 87.373825) (width 0.25) (layer "F.Cu") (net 10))
 (segment (start 84.315 90.424) (end 91.218036 90.424) (width 0.25) (layer "B.Cu") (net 10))
 (segment (start 95.065792 88.830207) (end 97.536 86.36) (width 0.25) (layer "B.Cu") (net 10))
 (arc (start 95.065792 88.830207) (mid 93.300426 90.009786) (end 91.218036 90.424) (width 0.25) (layer "B.Cu") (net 10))
 (segment (start 83.206789 82.695) (end 83.92521 82.695) (width 0.25) (layer "F.Cu") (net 7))
 (segment (start 84.074 83.312) (end 84.074 83.2575) (width 0.25) (layer "F.Cu") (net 7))
 (segment (start 82.379556 82.695) (end 83.206789 82.695) (width 0.25) (layer "F.Cu") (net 7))
 (segment (start 84.035462 83.164462) (end 83.82 82.949) (width 0.25) (layer "F.Cu") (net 7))
 (segment (start 80.6715 81.9875) (end 79.964 81.28) (width 0.25) (layer "F.Cu") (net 7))
 (segment (start 101.560792 88.900792) (end 104.14 91.48) (width 0.25) (layer "F.Cu") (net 7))
 (segment (start 85.09 93.472) (end 85.09 87.884) (width 0.25) (layer "F.Cu") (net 7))
 (segment (start 97.967001 82.695) (end 83.92521 82.695) (width 0.25) (layer "F.Cu") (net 7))
 (segment (start 99.967 84.694998) (end 99.967 85.053036) (width 0.25) (layer "F.Cu") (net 7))
 (segment (start 85.09 87.884) (end 82.804 85.598) (width 0.25) (layer "F.Cu") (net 7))
 (via (at 84.074 83.312) (size 0.8) (drill 0.4) (layers "F.Cu" "B.Cu") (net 7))
 (via (at 85.09 93.472) (size 0.8) (drill 0.4) (layers "F.Cu" "B.Cu") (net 7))
 (via (at 82.804 85.598) (size 0.8) (drill 0.4) (layers "F.Cu" "B.Cu") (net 7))
 (arc (start 99.967 84.694998) (mid 99.381213 83.280785) (end 97.967001 82.695) (width 0.25) (layer "F.Cu") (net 7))
 (arc (start 99.967 85.053036) (mid 100.381213 87.135426) (end 101.560792 88.900792) (width 0.25) (layer "F.Cu") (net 7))
 (arc (start 80.6715 81.9875) (mid 81.455162 82.511126) (end 82.379556 82.695) (width 0.25) (layer "F.Cu") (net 7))
 (arc (start 83.82 82.949) (mid 83.538656 82.761012) (end 83.206789 82.695) (width 0.25) (layer "F.Cu") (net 7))
 (arc (start 84.035462 83.164462) (mid 84.063984 83.207148) (end 84.074 83.2575) (width 0.25) (layer "F.Cu") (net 7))
 (arc (start 83.92521 82.695) (mid 83.787746 82.78685) (end 83.82 82.949) (width 0.25) (layer "F.Cu") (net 7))
 (segment (start 84.074 83.312) (end 83.16321 84.222789) (width 0.25) (layer "B.Cu") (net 7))
 (segment (start 82.804 85.598) (end 82.804 85.09) (width 0.25) (layer "B.Cu") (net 7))
 (segment (start 85.09 93.472) (end 83.566 94.996) (width 0.25) (layer "B.Cu") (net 7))
 (segment (start 79.886738 96.52) (end 74.676 96.52) (width 0.25) (layer "B.Cu") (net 7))
 (arc (start 83.566 94.996) (mid 81.87794 96.123925) (end 79.886738 96.52) (width 0.25) (layer "B.Cu") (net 7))
 (arc (start 83.16321 84.222789) (mid 82.897355 84.620669) (end 82.804 85.09) (width 0.25) (layer "B.Cu") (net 7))
 (segment (start 79.964 83.82) (end 80.0975 83.9535) (width 0.25) (layer "F.Cu") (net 8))
 (segment (start 94.435637 93.98) (end 97.632 93.98) (width 0.25) (layer "F.Cu") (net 8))
 (segment (start 80.419797 84.087) (end 89.430305 84.087) (width 0.25) (layer "F.Cu") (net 8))
 (segment (start 89.430305 84.087) (end 90.463152 85.119847) (width 0.25) (layer "F.Cu") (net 8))
 (segment (start 91.496 92.258) (end 92.357 93.119) (width 0.25) (layer "F.Cu") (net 8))
 (segment (start 91.496 87.613361) (end 91.496 92.258) (width 0.25) (layer "F.Cu") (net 8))
 (arc (start 80.0975 83.9535) (mid 80.245371 84.052304) (end 80.419797 84.087) (width 0.25) (layer "F.Cu") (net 8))
 (arc (start 90.463152 85.119847) (mid 91.227571 86.263881) (end 91.496 87.613361) (width 0.25) (layer "F.Cu") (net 8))
 (arc (start 92.357 93.119) (mid 93.310686 93.756233) (end 94.435637 93.98) (width 0.25) (layer "F.Cu") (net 8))
 (segment (start 104.79 85.83) (end 103.49 87.13) (width 0.25) (layer "B.Cu") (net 8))
 (segment (start 105.44 84.260761) (end 105.44 81.213238) (width 0.25) (layer "B.Cu") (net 8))
 (segment (start 99.177783 91.442216) (end 103.49 87.13) (width 0.25) (layer "B.Cu") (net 8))
 (segment (start 106.984 76.64) (end 107.474 76.64) (width 0.25) (layer "B.Cu") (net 8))
 (segment (start 98.544216 92.971783) (end 97.536 93.98) (width 0.25) (layer "B.Cu") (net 8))
 (segment (start 104.789999 78.343999) (end 106.147517 76.986482) (width 0.25) (layer "B.Cu") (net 8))
 (arc (start 106.984 76.64) (mid 106.531298 76.730047) (end 106.147517 76.986482) (width 0.25) (layer "B.Cu") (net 8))
 (arc (start 98.861 92.207) (mid 98.77867 92.620897) (end 98.544216 92.971783) (width 0.25) (layer "B.Cu") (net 8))
 (arc (start 105.44 84.260761) (mid 105.27107 85.110027) (end 104.79 85.83) (width 0.25) (layer "B.Cu") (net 8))
 (arc (start 104.789999 78.343999) (mid 104.52076 78.993999) (end 104.79 79.644) (width 0.25) (layer "B.Cu") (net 8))
 (arc (start 99.177783 91.442216) (mid 98.943329 91.793101) (end 98.861 92.207) (width 0.25) (layer "B.Cu") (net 8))
 (arc (start 104.79 79.644) (mid 105.27107 80.363972) (end 105.44 81.213238) (width 0.25) (layer "B.Cu") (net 8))
 (segment (start 84.315 88.646) (end 82.759087 87.090087) (width 0.25) (layer "F.Cu") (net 9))
 (segment (start 80.9965 86.36) (end 79.964 86.36) (width 0.25) (layer "F.Cu") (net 9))
 (via (at 84.315 88.646) (size 0.8) (drill 0.4) (layers "F.Cu" "B.Cu") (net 9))
 (arc (start 82.759087 87.090087) (mid 81.950405 86.549743) (end 80.9965 86.36) (width 0.25) (layer "F.Cu") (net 9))
 (segment (start 94.303792 87.052207) (end 97.446197 83.909802) (width 0.25) (layer "B.Cu") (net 9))
 (segment (start 90.456036 88.646) (end 84.315 88.646) (width 0.25) (layer "B.Cu") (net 9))
 (segment (start 98.063137 83.98) (end 104.14 83.98) (width 0.25) (layer "B.Cu") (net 9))
 (segment (start 97.676862 83.82) (end 97.663 83.82) (width 0.25) (layer "B.Cu") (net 9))
 (arc (start 94.303792 87.052207) (mid 92.538426 88.231786) (end 90.456036 88.646) (width 0.25) (layer "B.Cu") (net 9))
 (arc (start 97.87 83.9) (mid 97.958612 83.959208) (end 98.063137 83.98) (width 0.25) (layer "B.Cu") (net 9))
 (arc (start 97.87 83.9) (mid 97.781387 83.840791) (end 97.676862 83.82) (width 0.25) (layer "B.Cu") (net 9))
 (arc (start 97.663 83.82) (mid 97.545667 83.843338) (end 97.446197 83.909802) (width 0.25) (layer "B.Cu") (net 9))
 (segment (start 63.713869 72.209999) (end 72.114901 80.611031) (width 0.25) (layer "B.Cu") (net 18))
 (segment (start 62.748185 71.81) (end 62.1825 71.81) (width 0.25) (layer "B.Cu") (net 18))
 (segment (start 73.729935 81.28) (end 74.676 81.28) (width 0.25) (layer "B.Cu") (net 18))
 (arc (start 72.114901 80.611031) (mid 72.855884 81.10614) (end 73.729935 81.28) (width 0.25) (layer "B.Cu") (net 18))
 (arc (start 63.713869 72.209999) (mid 63.270809 71.913956) (end 62.748185 71.81) (width 0.25) (layer "B.Cu") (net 18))
 (segment (start 80.07875 79.08425) (end 78.9725 80.1905) (width 0.25) (layer "B.Cu") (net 19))
 (segment (start 97.028 80.01) (end 98.03 80.01) (width 0.25) (layer "B.Cu") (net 19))
 (segment (start 94.996 77.978) (end 82.749473 77.978) (width 0.25) (layer "B.Cu") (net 19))
 (segment (start 106.446 74.64) (end 107.474 74.64) (width 0.25) (layer "B.Cu") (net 19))
 (segment (start 104.691094 75.366905) (end 101.474941 78.583058) (width 0.25) (layer "B.Cu") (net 19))
 (arc (start 101.474941 78.583058) (mid 99.894388 79.639149) (end 98.03 80.01) (width 0.25) (layer "B.Cu") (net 19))
 (arc (start 106.446 74.64) (mid 105.496251 74.828916) (end 104.691094 75.366905) (width 0.25) (layer "B.Cu") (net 19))
 (arc (start 82.749473 77.978) (mid 81.304088 78.265505) (end 80.07875 79.08425) (width 0.25) (layer "B.Cu") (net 19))
 (arc (start 96.012 78.994) (mid 95.71442 78.275579) (end 94.996 77.978) (width 0.25) (layer "B.Cu") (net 19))
 (arc (start 96.012 78.994) (mid 96.309579 79.71242) (end 97.028 80.01) (width 0.25) (layer "B.Cu") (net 19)))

